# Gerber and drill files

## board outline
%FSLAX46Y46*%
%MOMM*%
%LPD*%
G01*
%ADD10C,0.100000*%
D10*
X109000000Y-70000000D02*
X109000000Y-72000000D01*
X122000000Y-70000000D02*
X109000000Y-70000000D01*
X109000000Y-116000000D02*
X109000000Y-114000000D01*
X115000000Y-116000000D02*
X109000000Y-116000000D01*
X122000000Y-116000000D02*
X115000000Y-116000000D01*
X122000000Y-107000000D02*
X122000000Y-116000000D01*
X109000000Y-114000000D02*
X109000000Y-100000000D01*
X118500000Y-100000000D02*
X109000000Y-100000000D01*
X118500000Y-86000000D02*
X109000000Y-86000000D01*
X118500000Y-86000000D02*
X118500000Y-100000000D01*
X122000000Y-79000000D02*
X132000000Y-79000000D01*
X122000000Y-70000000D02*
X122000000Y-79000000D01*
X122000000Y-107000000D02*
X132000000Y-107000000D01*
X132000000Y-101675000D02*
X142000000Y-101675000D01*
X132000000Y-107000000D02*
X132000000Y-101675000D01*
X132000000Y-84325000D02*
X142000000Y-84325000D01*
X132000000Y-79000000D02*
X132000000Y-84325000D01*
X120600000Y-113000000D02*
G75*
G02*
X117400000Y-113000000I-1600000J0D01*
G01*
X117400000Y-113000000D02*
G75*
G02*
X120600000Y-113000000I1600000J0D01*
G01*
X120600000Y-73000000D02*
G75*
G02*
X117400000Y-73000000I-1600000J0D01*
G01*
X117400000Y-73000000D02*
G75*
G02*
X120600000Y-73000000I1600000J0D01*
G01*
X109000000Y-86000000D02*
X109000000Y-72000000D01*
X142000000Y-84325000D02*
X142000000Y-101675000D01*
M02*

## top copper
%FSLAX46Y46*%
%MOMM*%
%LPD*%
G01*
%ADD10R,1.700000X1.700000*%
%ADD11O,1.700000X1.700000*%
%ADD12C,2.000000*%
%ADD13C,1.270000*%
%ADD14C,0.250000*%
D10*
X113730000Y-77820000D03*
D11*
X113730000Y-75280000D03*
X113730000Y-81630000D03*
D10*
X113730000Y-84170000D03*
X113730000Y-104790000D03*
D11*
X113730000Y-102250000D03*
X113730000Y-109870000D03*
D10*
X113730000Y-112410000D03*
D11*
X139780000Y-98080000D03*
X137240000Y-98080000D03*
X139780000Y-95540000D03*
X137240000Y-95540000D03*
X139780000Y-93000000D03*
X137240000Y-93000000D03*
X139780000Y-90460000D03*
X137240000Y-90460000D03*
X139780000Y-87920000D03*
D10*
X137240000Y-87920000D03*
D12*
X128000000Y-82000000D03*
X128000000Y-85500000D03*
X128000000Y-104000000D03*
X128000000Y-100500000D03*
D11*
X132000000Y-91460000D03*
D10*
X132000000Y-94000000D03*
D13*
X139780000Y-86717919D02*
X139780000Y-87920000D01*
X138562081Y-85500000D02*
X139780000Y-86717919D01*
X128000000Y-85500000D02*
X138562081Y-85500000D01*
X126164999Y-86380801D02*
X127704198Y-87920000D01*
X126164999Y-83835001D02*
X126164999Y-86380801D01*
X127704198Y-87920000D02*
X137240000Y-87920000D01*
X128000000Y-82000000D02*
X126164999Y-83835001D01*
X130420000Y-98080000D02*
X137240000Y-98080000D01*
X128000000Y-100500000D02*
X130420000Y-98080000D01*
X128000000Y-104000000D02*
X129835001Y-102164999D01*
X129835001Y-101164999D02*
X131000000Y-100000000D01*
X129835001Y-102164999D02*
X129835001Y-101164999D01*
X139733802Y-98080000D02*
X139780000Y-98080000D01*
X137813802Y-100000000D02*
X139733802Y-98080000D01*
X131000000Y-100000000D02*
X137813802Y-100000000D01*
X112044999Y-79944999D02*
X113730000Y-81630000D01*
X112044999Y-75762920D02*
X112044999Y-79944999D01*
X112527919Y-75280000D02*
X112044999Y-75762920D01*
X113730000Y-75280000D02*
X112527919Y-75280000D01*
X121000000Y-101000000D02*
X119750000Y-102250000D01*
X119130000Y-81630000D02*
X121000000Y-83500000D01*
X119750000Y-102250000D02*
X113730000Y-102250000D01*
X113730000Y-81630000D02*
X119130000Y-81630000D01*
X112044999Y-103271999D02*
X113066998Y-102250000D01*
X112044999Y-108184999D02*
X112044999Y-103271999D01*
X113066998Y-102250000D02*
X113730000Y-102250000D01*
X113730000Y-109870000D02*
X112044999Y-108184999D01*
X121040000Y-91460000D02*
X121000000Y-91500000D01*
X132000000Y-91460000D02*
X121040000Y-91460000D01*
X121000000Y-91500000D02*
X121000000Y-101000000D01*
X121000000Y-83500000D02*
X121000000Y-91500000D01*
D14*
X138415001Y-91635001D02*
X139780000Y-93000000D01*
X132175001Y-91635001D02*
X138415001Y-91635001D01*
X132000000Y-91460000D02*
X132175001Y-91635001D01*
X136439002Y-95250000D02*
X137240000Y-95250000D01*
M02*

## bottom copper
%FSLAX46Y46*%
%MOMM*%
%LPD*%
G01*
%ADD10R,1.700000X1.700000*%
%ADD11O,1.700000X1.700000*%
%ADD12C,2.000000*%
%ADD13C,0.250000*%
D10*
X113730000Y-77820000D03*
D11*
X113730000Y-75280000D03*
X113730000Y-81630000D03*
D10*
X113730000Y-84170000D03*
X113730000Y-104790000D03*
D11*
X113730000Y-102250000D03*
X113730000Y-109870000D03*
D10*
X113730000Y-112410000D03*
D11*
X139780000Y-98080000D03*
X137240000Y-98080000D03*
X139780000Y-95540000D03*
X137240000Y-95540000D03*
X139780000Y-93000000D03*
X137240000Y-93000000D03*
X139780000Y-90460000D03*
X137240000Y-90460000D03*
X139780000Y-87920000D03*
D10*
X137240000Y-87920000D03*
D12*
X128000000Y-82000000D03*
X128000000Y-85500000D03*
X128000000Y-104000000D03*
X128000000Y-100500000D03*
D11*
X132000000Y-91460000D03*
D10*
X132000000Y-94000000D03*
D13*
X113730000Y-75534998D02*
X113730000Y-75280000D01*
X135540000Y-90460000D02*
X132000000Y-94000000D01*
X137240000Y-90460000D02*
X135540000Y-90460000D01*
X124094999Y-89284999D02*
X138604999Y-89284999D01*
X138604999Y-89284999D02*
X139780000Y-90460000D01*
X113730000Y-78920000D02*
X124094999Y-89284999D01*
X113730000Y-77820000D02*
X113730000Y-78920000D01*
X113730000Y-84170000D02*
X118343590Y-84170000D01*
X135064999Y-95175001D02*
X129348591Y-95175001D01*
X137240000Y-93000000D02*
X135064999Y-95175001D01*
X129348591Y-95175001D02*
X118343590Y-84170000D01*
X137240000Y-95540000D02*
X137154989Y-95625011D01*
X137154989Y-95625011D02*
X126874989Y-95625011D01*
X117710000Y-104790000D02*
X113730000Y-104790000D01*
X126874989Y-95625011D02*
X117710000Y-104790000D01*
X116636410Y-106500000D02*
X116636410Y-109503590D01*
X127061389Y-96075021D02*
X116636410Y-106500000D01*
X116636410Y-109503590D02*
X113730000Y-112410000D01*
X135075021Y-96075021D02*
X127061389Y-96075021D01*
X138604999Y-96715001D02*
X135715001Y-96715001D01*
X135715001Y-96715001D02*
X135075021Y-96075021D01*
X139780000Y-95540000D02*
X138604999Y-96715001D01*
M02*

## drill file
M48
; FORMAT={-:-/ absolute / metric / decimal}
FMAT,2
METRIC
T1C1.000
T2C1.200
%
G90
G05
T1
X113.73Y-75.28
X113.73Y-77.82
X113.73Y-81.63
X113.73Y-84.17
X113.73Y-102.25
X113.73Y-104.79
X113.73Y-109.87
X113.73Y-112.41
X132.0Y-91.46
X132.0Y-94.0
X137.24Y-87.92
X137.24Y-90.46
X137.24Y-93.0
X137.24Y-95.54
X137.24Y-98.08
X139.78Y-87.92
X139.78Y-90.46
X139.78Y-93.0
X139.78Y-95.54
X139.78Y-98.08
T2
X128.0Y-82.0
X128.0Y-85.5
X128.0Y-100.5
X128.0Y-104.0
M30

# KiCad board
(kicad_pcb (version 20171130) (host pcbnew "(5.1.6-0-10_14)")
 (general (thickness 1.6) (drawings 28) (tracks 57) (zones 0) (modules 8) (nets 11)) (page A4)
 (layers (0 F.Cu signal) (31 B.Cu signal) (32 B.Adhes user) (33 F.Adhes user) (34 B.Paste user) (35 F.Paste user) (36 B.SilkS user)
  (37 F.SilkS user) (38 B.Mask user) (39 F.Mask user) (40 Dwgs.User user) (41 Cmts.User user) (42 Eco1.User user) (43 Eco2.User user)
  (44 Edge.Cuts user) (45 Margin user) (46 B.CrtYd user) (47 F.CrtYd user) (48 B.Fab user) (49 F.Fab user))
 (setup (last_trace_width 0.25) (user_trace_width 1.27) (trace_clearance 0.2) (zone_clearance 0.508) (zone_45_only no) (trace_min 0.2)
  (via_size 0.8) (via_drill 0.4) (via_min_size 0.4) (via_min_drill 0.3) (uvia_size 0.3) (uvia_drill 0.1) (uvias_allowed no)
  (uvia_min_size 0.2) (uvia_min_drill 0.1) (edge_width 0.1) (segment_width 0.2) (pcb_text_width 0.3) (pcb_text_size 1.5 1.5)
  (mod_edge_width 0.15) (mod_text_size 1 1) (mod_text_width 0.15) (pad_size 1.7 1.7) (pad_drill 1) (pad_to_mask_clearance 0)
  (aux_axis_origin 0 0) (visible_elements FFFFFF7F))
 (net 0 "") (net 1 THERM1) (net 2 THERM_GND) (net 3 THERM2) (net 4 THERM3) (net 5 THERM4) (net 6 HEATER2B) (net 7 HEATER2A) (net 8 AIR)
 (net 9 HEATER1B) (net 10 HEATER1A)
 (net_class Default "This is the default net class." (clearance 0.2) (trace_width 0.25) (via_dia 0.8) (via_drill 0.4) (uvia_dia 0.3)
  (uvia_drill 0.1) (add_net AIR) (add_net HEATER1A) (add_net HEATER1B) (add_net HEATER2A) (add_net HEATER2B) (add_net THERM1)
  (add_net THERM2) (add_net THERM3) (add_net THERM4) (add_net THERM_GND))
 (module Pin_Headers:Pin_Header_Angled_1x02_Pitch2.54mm (layer F.Cu) (at 113.73 77.82 180)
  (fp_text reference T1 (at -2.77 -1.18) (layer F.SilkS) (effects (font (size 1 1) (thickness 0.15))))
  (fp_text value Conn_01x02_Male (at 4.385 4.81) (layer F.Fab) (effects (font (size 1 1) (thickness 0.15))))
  (pad 1 thru_hole rect (at 0 0 180) (size 1.7 1.7) (drill 1) (layers *.Cu *.Mask) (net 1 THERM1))
  (pad 2 thru_hole oval (at 0 2.54 180) (size 1.7 1.7) (drill 1) (layers *.Cu *.Mask) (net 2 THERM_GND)))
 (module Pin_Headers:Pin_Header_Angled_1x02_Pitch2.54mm (layer F.Cu) (at 113.73 84.17 180)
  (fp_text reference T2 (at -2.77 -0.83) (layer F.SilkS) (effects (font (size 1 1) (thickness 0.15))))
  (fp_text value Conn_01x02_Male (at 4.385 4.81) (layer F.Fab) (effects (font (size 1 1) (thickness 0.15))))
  (pad 2 thru_hole oval (at 0 2.54 180) (size 1.7 1.7) (drill 1) (layers *.Cu *.Mask) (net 2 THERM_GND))
  (pad 1 thru_hole rect (at 0 0 180) (size 1.7 1.7) (drill 1) (layers *.Cu *.Mask) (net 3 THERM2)))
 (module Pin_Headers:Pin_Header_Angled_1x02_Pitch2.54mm (layer F.Cu) (at 113.73 104.79 180)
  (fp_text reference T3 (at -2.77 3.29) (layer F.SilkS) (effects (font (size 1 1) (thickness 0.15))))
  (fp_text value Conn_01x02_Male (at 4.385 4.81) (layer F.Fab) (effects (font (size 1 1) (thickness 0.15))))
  (pad 1 thru_hole rect (at 0 0 180) (size 1.7 1.7) (drill 1) (layers *.Cu *.Mask) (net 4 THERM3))
  (pad 2 thru_hole oval (at 0 2.54 180) (size 1.7 1.7) (drill 1) (layers *.Cu *.Mask) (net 2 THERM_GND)))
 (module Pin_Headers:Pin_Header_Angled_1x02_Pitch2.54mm (layer F.Cu) (at 113.73 112.41 180)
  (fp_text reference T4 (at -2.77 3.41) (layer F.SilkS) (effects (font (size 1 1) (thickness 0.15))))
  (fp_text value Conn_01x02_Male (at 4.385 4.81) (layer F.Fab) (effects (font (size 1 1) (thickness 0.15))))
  (pad 2 thru_hole oval (at 0 2.54 180) (size 1.7 1.7) (drill 1) (layers *.Cu *.Mask) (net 2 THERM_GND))
  (pad 1 thru_hole rect (at 0 0 180) (size 1.7 1.7) (drill 1) (layers *.Cu *.Mask) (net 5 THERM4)))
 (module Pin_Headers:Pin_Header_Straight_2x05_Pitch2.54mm (layer F.Cu) (at 137.24 87.92)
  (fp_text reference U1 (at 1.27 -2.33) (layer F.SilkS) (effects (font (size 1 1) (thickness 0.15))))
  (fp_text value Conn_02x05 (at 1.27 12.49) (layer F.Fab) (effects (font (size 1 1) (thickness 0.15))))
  (pad 10 thru_hole oval (at 2.54 10.16) (size 1.7 1.7) (drill 1) (layers *.Cu *.Mask) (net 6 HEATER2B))
  (pad 9 thru_hole oval (at 0 10.16) (size 1.7 1.7) (drill 1) (layers *.Cu *.Mask) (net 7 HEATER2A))
  (pad 8 thru_hole oval (at 2.54 7.62) (size 1.7 1.7) (drill 1) (layers *.Cu *.Mask) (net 5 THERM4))
  (pad 7 thru_hole oval (at 0 7.62) (size 1.7 1.7) (drill 1) (layers *.Cu *.Mask) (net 4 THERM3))
  (pad 6 thru_hole oval (at 2.54 5.08) (size 1.7 1.7) (drill 1) (layers *.Cu *.Mask) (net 2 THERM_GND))
  (pad 5 thru_hole oval (at 0 5.08) (size 1.7 1.7) (drill 1) (layers *.Cu *.Mask) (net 3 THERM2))
  (pad 4 thru_hole oval (at 2.54 2.54) (size 1.7 1.7) (drill 1) (layers *.Cu *.Mask) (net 1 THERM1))
  (pad 3 thru_hole oval (at 0 2.54) (size 1.7 1.7) (drill 1) (layers *.Cu *.Mask) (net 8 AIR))
  (pad 2 thru_hole oval (at 2.54 0) (size 1.7 1.7) (drill 1) (layers *.Cu *.Mask) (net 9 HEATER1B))
  (pad 1 thru_hole rect (at 0 0) (size 1.7 1.7) (drill 1) (layers *.Cu *.Mask) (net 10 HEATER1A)))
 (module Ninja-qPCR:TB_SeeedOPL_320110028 (layer F.Cu) (at 128 82 270)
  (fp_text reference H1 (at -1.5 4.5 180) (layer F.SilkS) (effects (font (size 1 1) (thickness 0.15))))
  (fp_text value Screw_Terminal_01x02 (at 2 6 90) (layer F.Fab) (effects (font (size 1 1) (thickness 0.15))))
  (pad 1 thru_hole circle (at 0 0 270) (size 2 2) (drill 1.2) (layers *.Cu *.Mask) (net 10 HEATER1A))
  (pad 2 thru_hole circle (at 3.5 0 270) (size 2 2) (drill 1.2) (layers *.Cu *.Mask) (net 9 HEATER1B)))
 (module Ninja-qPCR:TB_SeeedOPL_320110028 (layer F.Cu) (at 128 100.5 270)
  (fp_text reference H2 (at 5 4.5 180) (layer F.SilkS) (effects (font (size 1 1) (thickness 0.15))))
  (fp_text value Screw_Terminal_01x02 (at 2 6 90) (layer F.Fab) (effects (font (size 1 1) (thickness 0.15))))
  (pad 2 thru_hole circle (at 3.5 0 270) (size 2 2) (drill 1.2) (layers *.Cu *.Mask) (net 6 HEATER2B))
  (pad 1 thru_hole circle (at 0 0 270) (size 2 2) (drill 1.2) (layers *.Cu *.Mask) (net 7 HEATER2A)))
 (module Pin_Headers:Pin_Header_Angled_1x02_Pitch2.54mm (layer F.Cu) (at 132 94 180)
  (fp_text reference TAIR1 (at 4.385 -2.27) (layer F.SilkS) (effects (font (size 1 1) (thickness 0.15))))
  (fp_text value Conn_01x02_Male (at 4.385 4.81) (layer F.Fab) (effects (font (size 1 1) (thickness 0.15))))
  (pad 2 thru_hole oval (at 0 2.54 180) (size 1.7 1.7) (drill 1) (layers *.Cu *.Mask) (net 2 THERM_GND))
  (pad 1 thru_hole rect (at 0 0 180) (size 1.7 1.7) (drill 1) (layers *.Cu *.Mask) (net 8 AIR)))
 (gr_line (start 109 70) (end 109 72) (layer Edge.Cuts) (width 0.1))
 (gr_line (start 122 70) (end 109 70) (layer Edge.Cuts) (width 0.1))
 (gr_line (start 109 116) (end 109 114) (layer Edge.Cuts) (width 0.1))
 (gr_line (start 115 116) (end 109 116) (layer Edge.Cuts) (width 0.1))
 (gr_line (start 122 116) (end 115 116) (layer Edge.Cuts) (width 0.1))
 (gr_line (start 122 107) (end 122 116) (layer Edge.Cuts) (width 0.1))
 (gr_line (start 109 114) (end 109 100) (layer Edge.Cuts) (width 0.1))
 (gr_line (start 118.5 100) (end 109 100) (layer Edge.Cuts) (width 0.1))
 (gr_line (start 118.5 86) (end 109 86) (layer Edge.Cuts) (width 0.1))
 (gr_line (start 118.5 86) (end 118.5 100) (layer Edge.Cuts) (width 0.1))
 (gr_line (start 122 79) (end 132 79) (layer Edge.Cuts) (width 0.1))
 (gr_line (start 122 70) (end 122 79) (layer Edge.Cuts) (width 0.1))
 (gr_line (start 122 107) (end 132 107) (layer Edge.Cuts) (width 0.1))
 (gr_line (start 132 101.675) (end 142 101.675) (layer Edge.Cuts) (width 0.1))
 (gr_line (start 132 107) (end 132 101.675) (layer Edge.Cuts) (width 0.1))
 (gr_line (start 132 84.325) (end 142 84.325) (layer Edge.Cuts) (width 0.1))
 (gr_line (start 132 79) (end 132 84.325) (layer Edge.Cuts) (width 0.1))
 (gr_circle (center 119 113) (end 120.6 113) (layer Edge.Cuts) (width 0.1))
 (gr_circle (center 119 73) (end 120.6 73) (layer Edge.Cuts) (width 0.1))
 (gr_line (start 109 86) (end 109 72) (layer Edge.Cuts) (width 0.1))
 (gr_line (start 142 84.325) (end 142 101.675) (layer Edge.Cuts) (width 0.1))
 (segment (start 139.78 86.717919) (end 139.78 87.92) (width 1.27) (layer F.Cu) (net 9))
 (segment (start 138.562081 85.5) (end 139.78 86.717919) (width 1.27) (layer F.Cu) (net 9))
 (segment (start 128 85.5) (end 138.562081 85.5) (width 1.27) (layer F.Cu) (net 9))
 (segment (start 126.164999 86.380801) (end 127.704198 87.92) (width 1.27) (layer F.Cu) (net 10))
 (segment (start 126.164999 83.835001) (end 126.164999 86.380801) (width 1.27) (layer F.Cu) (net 10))
 (segment (start 127.704198 87.92) (end 137.24 87.92) (width 1.27) (layer F.Cu) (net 10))
 (segment (start 128 82) (end 126.164999 83.835001) (width 1.27) (layer F.Cu) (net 10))
 (segment (start 130.42 98.08) (end 137.24 98.08) (width 1.27) (layer F.Cu) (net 7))
 (segment (start 128 100.5) (end 130.42 98.08) (width 1.27) (layer F.Cu) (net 7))
 (segment (start 128 104) (end 129.835001 102.164999) (width 1.27) (layer F.Cu) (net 6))
 (segment (start 129.835001 101.164999) (end 131 100) (width 1.27) (layer F.Cu) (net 6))
 (segment (start 129.835001 102.164999) (end 129.835001 101.164999) (width 1.27) (layer F.Cu) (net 6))
 (segment (start 139.733802 98.08) (end 139.78 98.08) (width 1.27) (layer F.Cu) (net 6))
 (segment (start 137.813802 100) (end 139.733802 98.08) (width 1.27) (layer F.Cu) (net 6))
 (segment (start 131 100) (end 137.813802 100) (width 1.27) (layer F.Cu) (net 6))
 (segment (start 113.73 75.534998) (end 113.73 75.28) (width 0.25) (layer B.Cu) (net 2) (status 30))
 (segment (start 112.044999 79.944999) (end 113.73 81.63) (width 1.27) (layer F.Cu) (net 2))
 (segment (start 112.044999 75.76292) (end 112.044999 79.944999) (width 1.27) (layer F.Cu) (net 2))
 (segment (start 112.527919 75.28) (end 112.044999 75.76292) (width 1.27) (layer F.Cu) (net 2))
 (segment (start 113.73 75.28) (end 112.527919 75.28) (width 1.27) (layer F.Cu) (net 2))
 (segment (start 121 101) (end 119.75 102.25) (width 1.27) (layer F.Cu) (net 2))
 (segment (start 119.13 81.63) (end 121 83.5) (width 1.27) (layer F.Cu) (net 2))
 (segment (start 119.75 102.25) (end 113.73 102.25) (width 1.27) (layer F.Cu) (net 2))
 (segment (start 113.73 81.63) (end 119.13 81.63) (width 1.27) (layer F.Cu) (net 2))
 (segment (start 112.044999 103.271999) (end 113.066998 102.25) (width 1.27) (layer F.Cu) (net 2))
 (segment (start 112.044999 108.184999) (end 112.044999 103.271999) (width 1.27) (layer F.Cu) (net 2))
 (segment (start 113.066998 102.25) (end 113.73 102.25) (width 1.27) (layer F.Cu) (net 2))
 (segment (start 113.73 109.87) (end 112.044999 108.184999) (width 1.27) (layer F.Cu) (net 2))
 (segment (start 121.04 91.46) (end 121 91.5) (width 1.27) (layer F.Cu) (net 2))
 (segment (start 132 91.46) (end 121.04 91.46) (width 1.27) (layer F.Cu) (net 2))
 (segment (start 121 91.5) (end 121 101) (width 1.27) (layer F.Cu) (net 2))
 (segment (start 121 83.5) (end 121 91.5) (width 1.27) (layer F.Cu) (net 2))
 (segment (start 138.415001 91.635001) (end 139.78 93) (width 0.25) (layer F.Cu) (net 2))
 (segment (start 132.175001 91.635001) (end 138.415001 91.635001) (width 0.25) (layer F.Cu) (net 2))
 (segment (start 132 91.46) (end 132.175001 91.635001) (width 0.25) (layer F.Cu) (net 2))
 (segment (start 135.54 90.46) (end 132 94) (width 0.25) (layer B.Cu) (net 8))
 (segment (start 137.24 90.46) (end 135.54 90.46) (width 0.25) (layer B.Cu) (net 8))
 (segment (start 124.094999 89.284999) (end 138.604999 89.284999) (width 0.25) (layer B.Cu) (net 1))
 (segment (start 138.604999 89.284999) (end 139.78 90.46) (width 0.25) (layer B.Cu) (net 1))
 (segment (start 113.73 78.92) (end 124.094999 89.284999) (width 0.25) (layer B.Cu) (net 1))
 (segment (start 113.73 77.82) (end 113.73 78.92) (width 0.25) (layer B.Cu) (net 1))
 (segment (start 113.73 84.17) (end 118.34359 84.17) (width 0.25) (layer B.Cu) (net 3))
 (segment (start 135.064999 95.175001) (end 129.348591 95.175001) (width 0.25) (layer B.Cu) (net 3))
 (segment (start 137.24 93) (end 135.064999 95.175001) (width 0.25) (layer B.Cu) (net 3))
 (segment (start 129.348591 95.175001) (end 118.34359 84.17) (width 0.25) (layer B.Cu) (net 3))
 (segment (start 136.439002 95.25) (end 137.24 95.25) (width 0.25) (layer F.Cu) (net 4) (status 20))
 (segment (start 137.24 95.54) (end 137.154989 95.625011) (width 0.25) (layer B.Cu) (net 4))
 (segment (start 137.154989 95.625011) (end 126.874989 95.625011) (width 0.25) (layer B.Cu) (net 4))
 (segment (start 117.71 104.79) (end 113.73 104.79) (width 0.25) (layer B.Cu) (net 4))
 (segment (start 126.874989 95.625011) (end 117.71 104.79) (width 0.25) (layer B.Cu) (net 4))
 (segment (start 116.63641 106.5) (end 116.63641 109.50359) (width 0.25) (layer B.Cu) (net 5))
 (segment (start 127.061389 96.075021) (end 116.63641 106.5) (width 0.25) (layer B.Cu) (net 5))
 (segment (start 116.63641 109.50359) (end 113.73 112.41) (width 0.25) (layer B.Cu) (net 5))
 (segment (start 135.075021 96.075021) (end 127.061389 96.075021) (width 0.25) (layer B.Cu) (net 5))
 (segment (start 138.604999 96.715001) (end 135.715001 96.715001) (width 0.25) (layer B.Cu) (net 5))
 (segment (start 135.715001 96.715001) (end 135.075021 96.075021) (width 0.25) (layer B.Cu) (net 5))
 (segment (start 139.78 95.54) (end 138.604999 96.715001) (width 0.25) (layer B.Cu) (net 5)))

